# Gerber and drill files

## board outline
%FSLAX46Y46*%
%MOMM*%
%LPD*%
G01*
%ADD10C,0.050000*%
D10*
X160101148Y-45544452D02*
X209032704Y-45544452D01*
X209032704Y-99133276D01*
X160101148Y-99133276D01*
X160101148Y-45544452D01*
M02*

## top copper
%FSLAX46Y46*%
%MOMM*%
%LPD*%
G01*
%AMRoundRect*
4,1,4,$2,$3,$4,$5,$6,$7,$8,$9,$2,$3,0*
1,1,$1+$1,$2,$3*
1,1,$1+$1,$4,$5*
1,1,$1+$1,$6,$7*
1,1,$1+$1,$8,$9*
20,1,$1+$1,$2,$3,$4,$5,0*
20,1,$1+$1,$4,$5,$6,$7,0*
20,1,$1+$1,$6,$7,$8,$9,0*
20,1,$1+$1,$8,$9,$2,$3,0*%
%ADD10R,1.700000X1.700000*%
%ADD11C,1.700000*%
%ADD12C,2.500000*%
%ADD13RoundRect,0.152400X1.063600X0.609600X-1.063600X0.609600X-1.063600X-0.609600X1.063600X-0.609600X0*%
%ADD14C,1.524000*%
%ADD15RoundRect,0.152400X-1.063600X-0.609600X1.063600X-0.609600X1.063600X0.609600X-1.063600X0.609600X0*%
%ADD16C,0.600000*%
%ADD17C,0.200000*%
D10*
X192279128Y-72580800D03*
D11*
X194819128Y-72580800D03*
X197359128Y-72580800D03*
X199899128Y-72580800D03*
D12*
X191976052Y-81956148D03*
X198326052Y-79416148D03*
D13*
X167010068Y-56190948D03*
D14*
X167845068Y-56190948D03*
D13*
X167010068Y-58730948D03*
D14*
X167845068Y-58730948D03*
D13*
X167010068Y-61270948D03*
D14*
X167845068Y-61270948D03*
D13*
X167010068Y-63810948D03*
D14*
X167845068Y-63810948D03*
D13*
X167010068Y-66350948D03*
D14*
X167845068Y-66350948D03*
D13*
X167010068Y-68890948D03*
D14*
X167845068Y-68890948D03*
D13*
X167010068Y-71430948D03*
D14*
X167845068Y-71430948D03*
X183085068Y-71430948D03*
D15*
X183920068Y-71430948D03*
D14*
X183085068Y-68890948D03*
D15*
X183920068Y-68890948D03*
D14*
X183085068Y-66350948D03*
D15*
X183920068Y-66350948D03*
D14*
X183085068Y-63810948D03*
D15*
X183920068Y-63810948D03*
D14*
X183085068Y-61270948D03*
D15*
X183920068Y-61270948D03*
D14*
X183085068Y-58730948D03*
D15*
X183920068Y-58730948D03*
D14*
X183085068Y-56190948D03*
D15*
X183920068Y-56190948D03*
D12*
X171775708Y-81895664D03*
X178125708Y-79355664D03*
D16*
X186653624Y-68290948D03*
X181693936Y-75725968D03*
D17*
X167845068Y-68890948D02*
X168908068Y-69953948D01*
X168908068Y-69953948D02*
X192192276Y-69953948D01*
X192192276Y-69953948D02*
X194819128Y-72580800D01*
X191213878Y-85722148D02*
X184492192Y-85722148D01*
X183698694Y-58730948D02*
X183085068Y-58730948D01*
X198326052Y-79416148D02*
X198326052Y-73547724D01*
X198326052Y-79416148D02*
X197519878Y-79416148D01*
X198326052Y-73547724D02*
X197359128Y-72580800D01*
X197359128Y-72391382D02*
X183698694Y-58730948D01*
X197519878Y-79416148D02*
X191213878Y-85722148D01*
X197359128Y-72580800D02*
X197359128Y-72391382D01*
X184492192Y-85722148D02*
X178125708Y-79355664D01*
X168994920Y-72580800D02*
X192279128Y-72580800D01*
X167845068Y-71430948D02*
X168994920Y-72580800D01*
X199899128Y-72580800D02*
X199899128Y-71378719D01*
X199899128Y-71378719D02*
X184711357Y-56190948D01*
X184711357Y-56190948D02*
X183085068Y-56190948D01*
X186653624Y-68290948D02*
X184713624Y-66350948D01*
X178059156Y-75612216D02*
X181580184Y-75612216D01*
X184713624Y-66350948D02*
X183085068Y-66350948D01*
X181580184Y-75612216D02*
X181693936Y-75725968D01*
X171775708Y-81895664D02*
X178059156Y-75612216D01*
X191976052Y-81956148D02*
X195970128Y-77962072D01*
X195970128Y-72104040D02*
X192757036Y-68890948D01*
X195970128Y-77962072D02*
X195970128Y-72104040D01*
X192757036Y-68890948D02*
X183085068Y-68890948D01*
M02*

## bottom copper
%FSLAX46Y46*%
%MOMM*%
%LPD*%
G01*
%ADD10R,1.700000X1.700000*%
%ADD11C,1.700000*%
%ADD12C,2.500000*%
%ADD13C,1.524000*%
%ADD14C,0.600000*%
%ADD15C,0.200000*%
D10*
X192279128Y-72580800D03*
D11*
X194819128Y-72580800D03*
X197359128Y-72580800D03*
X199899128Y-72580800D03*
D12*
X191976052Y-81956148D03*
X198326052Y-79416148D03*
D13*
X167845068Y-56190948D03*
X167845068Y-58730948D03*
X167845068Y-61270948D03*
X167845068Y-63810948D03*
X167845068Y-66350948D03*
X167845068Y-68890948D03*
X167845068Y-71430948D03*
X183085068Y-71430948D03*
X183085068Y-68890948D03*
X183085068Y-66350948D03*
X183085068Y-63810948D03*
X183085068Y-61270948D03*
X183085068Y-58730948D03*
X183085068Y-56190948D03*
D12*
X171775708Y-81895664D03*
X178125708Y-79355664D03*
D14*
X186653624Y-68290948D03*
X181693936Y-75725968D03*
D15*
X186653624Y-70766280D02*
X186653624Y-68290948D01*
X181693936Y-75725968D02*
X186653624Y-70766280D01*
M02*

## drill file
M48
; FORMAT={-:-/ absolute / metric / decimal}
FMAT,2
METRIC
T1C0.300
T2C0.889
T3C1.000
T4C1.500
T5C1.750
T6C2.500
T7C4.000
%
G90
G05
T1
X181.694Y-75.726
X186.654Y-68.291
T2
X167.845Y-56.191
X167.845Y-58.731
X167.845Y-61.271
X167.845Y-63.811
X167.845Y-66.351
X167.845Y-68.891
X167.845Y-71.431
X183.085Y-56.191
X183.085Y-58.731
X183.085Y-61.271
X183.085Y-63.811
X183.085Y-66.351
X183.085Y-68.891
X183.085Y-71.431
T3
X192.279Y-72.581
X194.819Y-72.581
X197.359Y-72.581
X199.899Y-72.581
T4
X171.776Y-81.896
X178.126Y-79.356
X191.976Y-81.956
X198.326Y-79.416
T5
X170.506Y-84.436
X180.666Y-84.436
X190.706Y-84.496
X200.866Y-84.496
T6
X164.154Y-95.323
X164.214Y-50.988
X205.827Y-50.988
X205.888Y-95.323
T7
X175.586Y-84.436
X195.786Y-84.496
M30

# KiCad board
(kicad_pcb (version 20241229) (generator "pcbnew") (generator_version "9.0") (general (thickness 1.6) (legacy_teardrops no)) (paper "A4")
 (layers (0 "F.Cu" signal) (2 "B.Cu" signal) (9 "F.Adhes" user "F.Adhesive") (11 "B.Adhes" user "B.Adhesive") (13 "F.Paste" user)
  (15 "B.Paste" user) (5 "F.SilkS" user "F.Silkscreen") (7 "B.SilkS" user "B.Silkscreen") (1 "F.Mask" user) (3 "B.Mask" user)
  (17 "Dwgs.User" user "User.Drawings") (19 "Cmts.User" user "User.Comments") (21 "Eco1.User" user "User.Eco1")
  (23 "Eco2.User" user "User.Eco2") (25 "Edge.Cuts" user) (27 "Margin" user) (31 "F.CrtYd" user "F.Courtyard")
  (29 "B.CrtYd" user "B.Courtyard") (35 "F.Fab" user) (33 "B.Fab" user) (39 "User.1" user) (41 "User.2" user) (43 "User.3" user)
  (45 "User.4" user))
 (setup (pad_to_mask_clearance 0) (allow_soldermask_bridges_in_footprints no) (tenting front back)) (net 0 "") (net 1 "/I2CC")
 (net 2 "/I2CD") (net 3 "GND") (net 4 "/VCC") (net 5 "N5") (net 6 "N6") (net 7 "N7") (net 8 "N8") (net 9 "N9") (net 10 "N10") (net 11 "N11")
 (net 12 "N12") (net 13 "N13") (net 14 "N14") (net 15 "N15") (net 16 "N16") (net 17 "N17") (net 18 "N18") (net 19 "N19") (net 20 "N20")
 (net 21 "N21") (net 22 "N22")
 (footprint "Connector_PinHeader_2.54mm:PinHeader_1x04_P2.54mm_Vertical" (layer "F.Cu") (at 192.279128 72.5808 90)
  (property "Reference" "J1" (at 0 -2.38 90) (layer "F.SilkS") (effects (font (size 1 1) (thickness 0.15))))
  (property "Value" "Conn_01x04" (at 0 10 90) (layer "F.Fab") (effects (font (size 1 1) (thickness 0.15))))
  (pad "1" thru_hole rect (at 0 0 90) (size 1.7 1.7) (drill 1) (layers "*.Cu" "*.Mask") (remove_unused_layers no) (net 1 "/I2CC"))
  (pad "2" thru_hole circle (at 0 2.54 90) (size 1.7 1.7) (drill 1) (layers "*.Cu" "*.Mask") (remove_unused_layers no) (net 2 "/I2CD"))
  (pad "3" thru_hole circle (at 0 5.08 90) (size 1.7 1.7) (drill 1) (layers "*.Cu" "*.Mask") (remove_unused_layers no) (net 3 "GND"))
  (pad "4" thru_hole circle (at 0 7.62 90) (size 1.7 1.7) (drill 1) (layers "*.Cu" "*.Mask") (remove_unused_layers no) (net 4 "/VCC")))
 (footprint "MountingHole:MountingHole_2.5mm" (layer "F.Cu") (at 164.21406 50.988012)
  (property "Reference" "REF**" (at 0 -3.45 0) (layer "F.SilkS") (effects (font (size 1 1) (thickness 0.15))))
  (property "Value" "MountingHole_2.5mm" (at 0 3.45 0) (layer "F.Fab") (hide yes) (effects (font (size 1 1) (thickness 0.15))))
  (pad "" np_thru_hole circle (at 0 0) (size 2.5 2.5) (drill 2.5) (layers "*.Cu" "*.Mask")))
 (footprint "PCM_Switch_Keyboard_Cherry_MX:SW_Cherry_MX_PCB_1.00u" (layer "F.Cu") (at 195.786052 84.496148)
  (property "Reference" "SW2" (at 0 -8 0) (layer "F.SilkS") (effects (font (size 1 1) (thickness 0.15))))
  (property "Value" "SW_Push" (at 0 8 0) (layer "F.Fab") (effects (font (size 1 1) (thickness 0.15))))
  (pad "" np_thru_hole circle (at -5.08 0) (size 1.75 1.75) (drill 1.75) (layers "*.Cu" "*.Mask"))
  (pad "" np_thru_hole circle (at 0 0) (size 4 4) (drill 4) (layers "*.Cu" "*.Mask"))
  (pad "" np_thru_hole circle (at 5.08 0) (size 1.75 1.75) (drill 1.75) (layers "*.Cu" "*.Mask"))
  (pad "1" thru_hole circle (at -3.81 -2.54) (size 2.5 2.5) (drill 1.5) (layers "*.Cu" "*.Mask") (remove_unused_layers no) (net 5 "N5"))
  (pad "2" thru_hole circle (at 2.54 -5.08) (size 2.5 2.5) (drill 1.5) (layers "*.Cu" "*.Mask") (remove_unused_layers no) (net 3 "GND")))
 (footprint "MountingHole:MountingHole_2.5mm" (layer "F.Cu") (at 164.153576 95.322784)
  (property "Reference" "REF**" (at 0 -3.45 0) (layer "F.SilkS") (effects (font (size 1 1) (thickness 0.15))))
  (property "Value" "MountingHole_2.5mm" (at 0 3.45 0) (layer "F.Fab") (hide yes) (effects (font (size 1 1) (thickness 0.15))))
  (pad "" np_thru_hole circle (at 0 0) (size 2.5 2.5) (drill 2.5) (layers "*.Cu" "*.Mask")))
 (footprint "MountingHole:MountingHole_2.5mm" (layer "F.Cu") (at 205.827052 50.988012)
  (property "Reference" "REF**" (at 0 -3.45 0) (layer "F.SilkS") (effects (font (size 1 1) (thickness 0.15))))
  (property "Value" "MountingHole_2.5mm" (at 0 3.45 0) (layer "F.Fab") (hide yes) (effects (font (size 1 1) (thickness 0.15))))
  (pad "" np_thru_hole circle (at 0 0) (size 2.5 2.5) (drill 2.5) (layers "*.Cu" "*.Mask")))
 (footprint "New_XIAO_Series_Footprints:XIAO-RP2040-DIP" (layer "F.Cu") (at 175.465068 63.810948 90)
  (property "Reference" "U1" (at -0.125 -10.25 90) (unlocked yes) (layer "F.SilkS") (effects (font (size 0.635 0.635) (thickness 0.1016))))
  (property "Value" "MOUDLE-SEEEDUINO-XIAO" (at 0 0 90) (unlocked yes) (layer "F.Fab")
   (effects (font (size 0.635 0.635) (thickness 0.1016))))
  (pad "1" smd roundrect (at 7.62 -8.455 180) (size 2.432 1.524) (layers "F.Cu" "F.Mask") (roundrect_rratio 0.1) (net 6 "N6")
   (thermal_bridge_angle 45))
  (pad "1" thru_hole circle (at 7.62 -7.62 180) (size 1.524 1.524) (drill 0.889) (layers "*.Cu" "*.Mask") (remove_unused_layers no)
   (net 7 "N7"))
  (pad "2" smd roundrect (at 5.08 -8.455 180) (size 2.432 1.524) (layers "F.Cu" "F.Mask") (roundrect_rratio 0.1) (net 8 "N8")
   (thermal_bridge_angle 45))
  (pad "2" thru_hole circle (at 5.08 -7.62 180) (size 1.524 1.524) (drill 0.889) (layers "*.Cu" "*.Mask") (remove_unused_layers no)
   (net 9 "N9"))
  (pad "3" smd roundrect (at 2.54 -8.455 180) (size 2.432 1.524) (layers "F.Cu" "F.Mask") (roundrect_rratio 0.1) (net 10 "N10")
   (thermal_bridge_angle 45))
  (pad "3" thru_hole circle (at 2.54 -7.62 180) (size 1.524 1.524) (drill 0.889) (layers "*.Cu" "*.Mask") (remove_unused_layers no)
   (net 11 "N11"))
  (pad "4" smd roundrect (at 0 -8.455 180) (size 2.432 1.524) (layers "F.Cu" "F.Mask") (roundrect_rratio 0.1) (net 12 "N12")
   (thermal_bridge_angle 45))
  (pad "4" thru_hole circle (at 0 -7.62 180) (size 1.524 1.524) (drill 0.889) (layers "*.Cu" "*.Mask") (remove_unused_layers no)
   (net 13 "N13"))
  (pad "5" smd roundrect (at -2.54 -8.455 180) (size 2.432 1.524) (layers "F.Cu" "F.Mask") (roundrect_rratio 0.1) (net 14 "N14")
   (thermal_bridge_angle 45))
  (pad "5" thru_hole circle (at -2.54 -7.62 180) (size 1.524 1.524) (drill 0.889) (layers "*.Cu" "*.Mask") (remove_unused_layers no)
   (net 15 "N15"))
  (pad "6" smd roundrect (at -5.08 -8.455 180) (size 2.432 1.524) (layers "F.Cu" "F.Mask") (roundrect_rratio 0.1) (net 2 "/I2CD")
   (thermal_bridge_angle 45))
  (pad "6" thru_hole circle (at -5.08 -7.62 180) (size 1.524 1.524) (drill 0.889) (layers "*.Cu" "*.Mask") (remove_unused_layers no)
   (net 2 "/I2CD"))
  (pad "7" smd roundrect (at -7.62 -8.455 180) (size 2.432 1.524) (layers "F.Cu" "F.Mask") (roundrect_rratio 0.1) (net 1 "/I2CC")
   (thermal_bridge_angle 45))
  (pad "7" thru_hole circle (at -7.62 -7.62 180) (size 1.524 1.524) (drill 0.889) (layers "*.Cu" "*.Mask") (remove_unused_layers no)
   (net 1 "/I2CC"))
  (pad "8" thru_hole circle (at -7.62 7.62) (size 1.524 1.524) (drill 0.889) (layers "*.Cu" "*.Mask") (remove_unused_layers no)
   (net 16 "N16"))
  (pad "8" smd roundrect (at -7.62 8.455) (size 2.432 1.524) (layers "F.Cu" "F.Mask") (roundrect_rratio 0.1) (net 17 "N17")
   (thermal_bridge_angle 45))
  (pad "9" thru_hole circle (at -5.08 7.62) (size 1.524 1.524) (drill 0.889) (layers "*.Cu" "*.Mask") (remove_unused_layers no) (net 5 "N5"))
  (pad "9" smd roundrect (at -5.08 8.455) (size 2.432 1.524) (layers "F.Cu" "F.Mask") (roundrect_rratio 0.1) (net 5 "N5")
   (thermal_bridge_angle 45))
  (pad "10" thru_hole circle (at -2.54 7.62) (size 1.524 1.524) (drill 0.889) (layers "*.Cu" "*.Mask") (remove_unused_layers no)
   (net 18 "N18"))
  (pad "10" smd roundrect (at -2.54 8.455) (size 2.432 1.524) (layers "F.Cu" "F.Mask") (roundrect_rratio 0.1) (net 18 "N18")
   (thermal_bridge_angle 45))
  (pad "11" thru_hole circle (at 0 7.62) (size 1.524 1.524) (drill 0.889) (layers "*.Cu" "*.Mask") (remove_unused_layers no) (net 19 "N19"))
  (pad "11" smd roundrect (at 0 8.455) (size 2.432 1.524) (layers "F.Cu" "F.Mask") (roundrect_rratio 0.1) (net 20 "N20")
   (thermal_bridge_angle 45))
  (pad "12" thru_hole circle (at 2.54 7.62) (size 1.524 1.524) (drill 0.889) (layers "*.Cu" "*.Mask") (remove_unused_layers no)
   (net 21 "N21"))
  (pad "12" smd roundrect (at 2.54 8.455) (size 2.432 1.524) (layers "F.Cu" "F.Mask") (roundrect_rratio 0.1) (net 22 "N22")
   (thermal_bridge_angle 45))
  (pad "13" thru_hole circle (at 5.08 7.62) (size 1.524 1.524) (drill 0.889) (layers "*.Cu" "*.Mask") (remove_unused_layers no)
   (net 3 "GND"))
  (pad "13" smd roundrect (at 5.08 8.455) (size 2.432 1.524) (layers "F.Cu" "F.Mask") (roundrect_rratio 0.1) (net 3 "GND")
   (thermal_bridge_angle 45))
  (pad "14" thru_hole circle (at 7.62 7.62) (size 1.524 1.524) (drill 0.889) (layers "*.Cu" "*.Mask") (remove_unused_layers no)
   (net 4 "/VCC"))
  (pad "14" smd roundrect (at 7.62 8.455) (size 2.432 1.524) (layers "F.Cu" "F.Mask") (roundrect_rratio 0.1) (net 4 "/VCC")
   (thermal_bridge_angle 45)))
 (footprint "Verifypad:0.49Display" (layer "F.Cu") (at 193.609284 63.20578)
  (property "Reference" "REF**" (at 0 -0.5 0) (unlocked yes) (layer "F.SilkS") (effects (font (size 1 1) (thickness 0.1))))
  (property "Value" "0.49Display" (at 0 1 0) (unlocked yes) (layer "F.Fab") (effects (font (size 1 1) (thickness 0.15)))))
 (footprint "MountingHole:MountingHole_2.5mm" (layer "F.Cu") (at 205.887536 95.322784)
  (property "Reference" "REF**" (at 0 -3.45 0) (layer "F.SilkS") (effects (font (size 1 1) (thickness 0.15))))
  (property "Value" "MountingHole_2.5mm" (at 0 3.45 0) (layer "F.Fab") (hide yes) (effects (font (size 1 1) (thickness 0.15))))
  (pad "" np_thru_hole circle (at 0 0) (size 2.5 2.5) (drill 2.5) (layers "*.Cu" "*.Mask")))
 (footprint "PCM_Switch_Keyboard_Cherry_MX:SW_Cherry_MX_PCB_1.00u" (layer "F.Cu") (at 175.585708 84.435664)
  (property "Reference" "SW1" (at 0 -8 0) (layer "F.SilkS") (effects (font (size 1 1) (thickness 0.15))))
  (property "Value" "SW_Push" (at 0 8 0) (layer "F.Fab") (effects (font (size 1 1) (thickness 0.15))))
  (pad "" np_thru_hole circle (at -5.08 0) (size 1.75 1.75) (drill 1.75) (layers "*.Cu" "*.Mask"))
  (pad "" np_thru_hole circle (at 0 0) (size 4 4) (drill 4) (layers "*.Cu" "*.Mask"))
  (pad "" np_thru_hole circle (at 5.08 0) (size 1.75 1.75) (drill 1.75) (layers "*.Cu" "*.Mask"))
  (pad "1" thru_hole circle (at -3.81 -2.54) (size 2.5 2.5) (drill 1.5) (layers "*.Cu" "*.Mask") (remove_unused_layers no) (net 18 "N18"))
  (pad "2" thru_hole circle (at 2.54 -5.08) (size 2.5 2.5) (drill 1.5) (layers "*.Cu" "*.Mask") (remove_unused_layers no) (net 3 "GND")))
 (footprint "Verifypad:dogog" (layer "B.Cu") (at 175.734887 92.160269 180)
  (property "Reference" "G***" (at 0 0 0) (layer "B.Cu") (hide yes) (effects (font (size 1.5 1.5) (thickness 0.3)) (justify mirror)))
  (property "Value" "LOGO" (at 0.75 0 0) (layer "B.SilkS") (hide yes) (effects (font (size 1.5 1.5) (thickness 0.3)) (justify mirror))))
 (gr_rect (start 160.101148 45.544452) (end 209.032704 99.133276) (stroke (width 0.05) (type default)) (fill no) (layer "Edge.Cuts"))
 (segment (start 167.845068 68.890948) (end 168.908068 69.953948) (width 0.2) (layer "F.Cu") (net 2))
 (segment (start 168.908068 69.953948) (end 192.192276 69.953948) (width 0.2) (layer "F.Cu") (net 2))
 (segment (start 192.192276 69.953948) (end 194.819128 72.5808) (width 0.2) (layer "F.Cu") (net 2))
 (segment (start 191.213878 85.722148) (end 184.492192 85.722148) (width 0.2) (layer "F.Cu") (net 3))
 (segment (start 183.698694 58.730948) (end 183.085068 58.730948) (width 0.2) (layer "F.Cu") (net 3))
 (segment (start 198.326052 79.416148) (end 198.326052 73.547724) (width 0.2) (layer "F.Cu") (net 3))
 (segment (start 198.326052 79.416148) (end 197.519878 79.416148) (width 0.2) (layer "F.Cu") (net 3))
 (segment (start 198.326052 73.547724) (end 197.359128 72.5808) (width 0.2) (layer "F.Cu") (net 3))
 (segment (start 197.359128 72.391382) (end 183.698694 58.730948) (width 0.2) (layer "F.Cu") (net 3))
 (segment (start 197.519878 79.416148) (end 191.213878 85.722148) (width 0.2) (layer "F.Cu") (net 3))
 (segment (start 197.359128 72.5808) (end 197.359128 72.391382) (width 0.2) (layer "F.Cu") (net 3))
 (segment (start 184.492192 85.722148) (end 178.125708 79.355664) (width 0.2) (layer "F.Cu") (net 3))
 (segment (start 168.99492 72.5808) (end 192.279128 72.5808) (width 0.2) (layer "F.Cu") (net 1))
 (segment (start 167.845068 71.430948) (end 168.99492 72.5808) (width 0.2) (layer "F.Cu") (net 1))
 (segment (start 199.899128 72.5808) (end 199.899128 71.378719) (width 0.2) (layer "F.Cu") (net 4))
 (segment (start 199.899128 71.378719) (end 184.711357 56.190948) (width 0.2) (layer "F.Cu") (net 4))
 (segment (start 184.711357 56.190948) (end 183.085068 56.190948) (width 0.2) (layer "F.Cu") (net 4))
 (segment (start 186.653624 68.290948) (end 184.713624 66.350948) (width 0.2) (layer "F.Cu") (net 18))
 (segment (start 178.059156 75.612216) (end 181.580184 75.612216) (width 0.2) (layer "F.Cu") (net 18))
 (segment (start 184.713624 66.350948) (end 183.085068 66.350948) (width 0.2) (layer "F.Cu") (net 18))
 (segment (start 181.580184 75.612216) (end 181.693936 75.725968) (width 0.2) (layer "F.Cu") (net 18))
 (segment (start 171.775708 81.895664) (end 178.059156 75.612216) (width 0.2) (layer "F.Cu") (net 18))
 (via (at 186.653624 68.290948) (size 0.6) (drill 0.3) (layers "F.Cu" "B.Cu") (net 18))
 (via (at 181.693936 75.725968) (size 0.6) (drill 0.3) (layers "F.Cu" "B.Cu") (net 18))
 (segment (start 186.653624 70.76628) (end 186.653624 68.290948) (width 0.2) (layer "B.Cu") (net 18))
 (segment (start 181.693936 75.725968) (end 186.653624 70.76628) (width 0.2) (layer "B.Cu") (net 18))
 (segment (start 191.976052 81.956148) (end 195.970128 77.962072) (width 0.2) (layer "F.Cu") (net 5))
 (segment (start 195.970128 72.10404) (end 192.757036 68.890948) (width 0.2) (layer "F.Cu") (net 5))
 (segment (start 195.970128 77.962072) (end 195.970128 72.10404) (width 0.2) (layer "F.Cu") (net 5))
 (segment (start 192.757036 68.890948) (end 183.085068 68.890948) (width 0.2) (layer "F.Cu") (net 5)))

